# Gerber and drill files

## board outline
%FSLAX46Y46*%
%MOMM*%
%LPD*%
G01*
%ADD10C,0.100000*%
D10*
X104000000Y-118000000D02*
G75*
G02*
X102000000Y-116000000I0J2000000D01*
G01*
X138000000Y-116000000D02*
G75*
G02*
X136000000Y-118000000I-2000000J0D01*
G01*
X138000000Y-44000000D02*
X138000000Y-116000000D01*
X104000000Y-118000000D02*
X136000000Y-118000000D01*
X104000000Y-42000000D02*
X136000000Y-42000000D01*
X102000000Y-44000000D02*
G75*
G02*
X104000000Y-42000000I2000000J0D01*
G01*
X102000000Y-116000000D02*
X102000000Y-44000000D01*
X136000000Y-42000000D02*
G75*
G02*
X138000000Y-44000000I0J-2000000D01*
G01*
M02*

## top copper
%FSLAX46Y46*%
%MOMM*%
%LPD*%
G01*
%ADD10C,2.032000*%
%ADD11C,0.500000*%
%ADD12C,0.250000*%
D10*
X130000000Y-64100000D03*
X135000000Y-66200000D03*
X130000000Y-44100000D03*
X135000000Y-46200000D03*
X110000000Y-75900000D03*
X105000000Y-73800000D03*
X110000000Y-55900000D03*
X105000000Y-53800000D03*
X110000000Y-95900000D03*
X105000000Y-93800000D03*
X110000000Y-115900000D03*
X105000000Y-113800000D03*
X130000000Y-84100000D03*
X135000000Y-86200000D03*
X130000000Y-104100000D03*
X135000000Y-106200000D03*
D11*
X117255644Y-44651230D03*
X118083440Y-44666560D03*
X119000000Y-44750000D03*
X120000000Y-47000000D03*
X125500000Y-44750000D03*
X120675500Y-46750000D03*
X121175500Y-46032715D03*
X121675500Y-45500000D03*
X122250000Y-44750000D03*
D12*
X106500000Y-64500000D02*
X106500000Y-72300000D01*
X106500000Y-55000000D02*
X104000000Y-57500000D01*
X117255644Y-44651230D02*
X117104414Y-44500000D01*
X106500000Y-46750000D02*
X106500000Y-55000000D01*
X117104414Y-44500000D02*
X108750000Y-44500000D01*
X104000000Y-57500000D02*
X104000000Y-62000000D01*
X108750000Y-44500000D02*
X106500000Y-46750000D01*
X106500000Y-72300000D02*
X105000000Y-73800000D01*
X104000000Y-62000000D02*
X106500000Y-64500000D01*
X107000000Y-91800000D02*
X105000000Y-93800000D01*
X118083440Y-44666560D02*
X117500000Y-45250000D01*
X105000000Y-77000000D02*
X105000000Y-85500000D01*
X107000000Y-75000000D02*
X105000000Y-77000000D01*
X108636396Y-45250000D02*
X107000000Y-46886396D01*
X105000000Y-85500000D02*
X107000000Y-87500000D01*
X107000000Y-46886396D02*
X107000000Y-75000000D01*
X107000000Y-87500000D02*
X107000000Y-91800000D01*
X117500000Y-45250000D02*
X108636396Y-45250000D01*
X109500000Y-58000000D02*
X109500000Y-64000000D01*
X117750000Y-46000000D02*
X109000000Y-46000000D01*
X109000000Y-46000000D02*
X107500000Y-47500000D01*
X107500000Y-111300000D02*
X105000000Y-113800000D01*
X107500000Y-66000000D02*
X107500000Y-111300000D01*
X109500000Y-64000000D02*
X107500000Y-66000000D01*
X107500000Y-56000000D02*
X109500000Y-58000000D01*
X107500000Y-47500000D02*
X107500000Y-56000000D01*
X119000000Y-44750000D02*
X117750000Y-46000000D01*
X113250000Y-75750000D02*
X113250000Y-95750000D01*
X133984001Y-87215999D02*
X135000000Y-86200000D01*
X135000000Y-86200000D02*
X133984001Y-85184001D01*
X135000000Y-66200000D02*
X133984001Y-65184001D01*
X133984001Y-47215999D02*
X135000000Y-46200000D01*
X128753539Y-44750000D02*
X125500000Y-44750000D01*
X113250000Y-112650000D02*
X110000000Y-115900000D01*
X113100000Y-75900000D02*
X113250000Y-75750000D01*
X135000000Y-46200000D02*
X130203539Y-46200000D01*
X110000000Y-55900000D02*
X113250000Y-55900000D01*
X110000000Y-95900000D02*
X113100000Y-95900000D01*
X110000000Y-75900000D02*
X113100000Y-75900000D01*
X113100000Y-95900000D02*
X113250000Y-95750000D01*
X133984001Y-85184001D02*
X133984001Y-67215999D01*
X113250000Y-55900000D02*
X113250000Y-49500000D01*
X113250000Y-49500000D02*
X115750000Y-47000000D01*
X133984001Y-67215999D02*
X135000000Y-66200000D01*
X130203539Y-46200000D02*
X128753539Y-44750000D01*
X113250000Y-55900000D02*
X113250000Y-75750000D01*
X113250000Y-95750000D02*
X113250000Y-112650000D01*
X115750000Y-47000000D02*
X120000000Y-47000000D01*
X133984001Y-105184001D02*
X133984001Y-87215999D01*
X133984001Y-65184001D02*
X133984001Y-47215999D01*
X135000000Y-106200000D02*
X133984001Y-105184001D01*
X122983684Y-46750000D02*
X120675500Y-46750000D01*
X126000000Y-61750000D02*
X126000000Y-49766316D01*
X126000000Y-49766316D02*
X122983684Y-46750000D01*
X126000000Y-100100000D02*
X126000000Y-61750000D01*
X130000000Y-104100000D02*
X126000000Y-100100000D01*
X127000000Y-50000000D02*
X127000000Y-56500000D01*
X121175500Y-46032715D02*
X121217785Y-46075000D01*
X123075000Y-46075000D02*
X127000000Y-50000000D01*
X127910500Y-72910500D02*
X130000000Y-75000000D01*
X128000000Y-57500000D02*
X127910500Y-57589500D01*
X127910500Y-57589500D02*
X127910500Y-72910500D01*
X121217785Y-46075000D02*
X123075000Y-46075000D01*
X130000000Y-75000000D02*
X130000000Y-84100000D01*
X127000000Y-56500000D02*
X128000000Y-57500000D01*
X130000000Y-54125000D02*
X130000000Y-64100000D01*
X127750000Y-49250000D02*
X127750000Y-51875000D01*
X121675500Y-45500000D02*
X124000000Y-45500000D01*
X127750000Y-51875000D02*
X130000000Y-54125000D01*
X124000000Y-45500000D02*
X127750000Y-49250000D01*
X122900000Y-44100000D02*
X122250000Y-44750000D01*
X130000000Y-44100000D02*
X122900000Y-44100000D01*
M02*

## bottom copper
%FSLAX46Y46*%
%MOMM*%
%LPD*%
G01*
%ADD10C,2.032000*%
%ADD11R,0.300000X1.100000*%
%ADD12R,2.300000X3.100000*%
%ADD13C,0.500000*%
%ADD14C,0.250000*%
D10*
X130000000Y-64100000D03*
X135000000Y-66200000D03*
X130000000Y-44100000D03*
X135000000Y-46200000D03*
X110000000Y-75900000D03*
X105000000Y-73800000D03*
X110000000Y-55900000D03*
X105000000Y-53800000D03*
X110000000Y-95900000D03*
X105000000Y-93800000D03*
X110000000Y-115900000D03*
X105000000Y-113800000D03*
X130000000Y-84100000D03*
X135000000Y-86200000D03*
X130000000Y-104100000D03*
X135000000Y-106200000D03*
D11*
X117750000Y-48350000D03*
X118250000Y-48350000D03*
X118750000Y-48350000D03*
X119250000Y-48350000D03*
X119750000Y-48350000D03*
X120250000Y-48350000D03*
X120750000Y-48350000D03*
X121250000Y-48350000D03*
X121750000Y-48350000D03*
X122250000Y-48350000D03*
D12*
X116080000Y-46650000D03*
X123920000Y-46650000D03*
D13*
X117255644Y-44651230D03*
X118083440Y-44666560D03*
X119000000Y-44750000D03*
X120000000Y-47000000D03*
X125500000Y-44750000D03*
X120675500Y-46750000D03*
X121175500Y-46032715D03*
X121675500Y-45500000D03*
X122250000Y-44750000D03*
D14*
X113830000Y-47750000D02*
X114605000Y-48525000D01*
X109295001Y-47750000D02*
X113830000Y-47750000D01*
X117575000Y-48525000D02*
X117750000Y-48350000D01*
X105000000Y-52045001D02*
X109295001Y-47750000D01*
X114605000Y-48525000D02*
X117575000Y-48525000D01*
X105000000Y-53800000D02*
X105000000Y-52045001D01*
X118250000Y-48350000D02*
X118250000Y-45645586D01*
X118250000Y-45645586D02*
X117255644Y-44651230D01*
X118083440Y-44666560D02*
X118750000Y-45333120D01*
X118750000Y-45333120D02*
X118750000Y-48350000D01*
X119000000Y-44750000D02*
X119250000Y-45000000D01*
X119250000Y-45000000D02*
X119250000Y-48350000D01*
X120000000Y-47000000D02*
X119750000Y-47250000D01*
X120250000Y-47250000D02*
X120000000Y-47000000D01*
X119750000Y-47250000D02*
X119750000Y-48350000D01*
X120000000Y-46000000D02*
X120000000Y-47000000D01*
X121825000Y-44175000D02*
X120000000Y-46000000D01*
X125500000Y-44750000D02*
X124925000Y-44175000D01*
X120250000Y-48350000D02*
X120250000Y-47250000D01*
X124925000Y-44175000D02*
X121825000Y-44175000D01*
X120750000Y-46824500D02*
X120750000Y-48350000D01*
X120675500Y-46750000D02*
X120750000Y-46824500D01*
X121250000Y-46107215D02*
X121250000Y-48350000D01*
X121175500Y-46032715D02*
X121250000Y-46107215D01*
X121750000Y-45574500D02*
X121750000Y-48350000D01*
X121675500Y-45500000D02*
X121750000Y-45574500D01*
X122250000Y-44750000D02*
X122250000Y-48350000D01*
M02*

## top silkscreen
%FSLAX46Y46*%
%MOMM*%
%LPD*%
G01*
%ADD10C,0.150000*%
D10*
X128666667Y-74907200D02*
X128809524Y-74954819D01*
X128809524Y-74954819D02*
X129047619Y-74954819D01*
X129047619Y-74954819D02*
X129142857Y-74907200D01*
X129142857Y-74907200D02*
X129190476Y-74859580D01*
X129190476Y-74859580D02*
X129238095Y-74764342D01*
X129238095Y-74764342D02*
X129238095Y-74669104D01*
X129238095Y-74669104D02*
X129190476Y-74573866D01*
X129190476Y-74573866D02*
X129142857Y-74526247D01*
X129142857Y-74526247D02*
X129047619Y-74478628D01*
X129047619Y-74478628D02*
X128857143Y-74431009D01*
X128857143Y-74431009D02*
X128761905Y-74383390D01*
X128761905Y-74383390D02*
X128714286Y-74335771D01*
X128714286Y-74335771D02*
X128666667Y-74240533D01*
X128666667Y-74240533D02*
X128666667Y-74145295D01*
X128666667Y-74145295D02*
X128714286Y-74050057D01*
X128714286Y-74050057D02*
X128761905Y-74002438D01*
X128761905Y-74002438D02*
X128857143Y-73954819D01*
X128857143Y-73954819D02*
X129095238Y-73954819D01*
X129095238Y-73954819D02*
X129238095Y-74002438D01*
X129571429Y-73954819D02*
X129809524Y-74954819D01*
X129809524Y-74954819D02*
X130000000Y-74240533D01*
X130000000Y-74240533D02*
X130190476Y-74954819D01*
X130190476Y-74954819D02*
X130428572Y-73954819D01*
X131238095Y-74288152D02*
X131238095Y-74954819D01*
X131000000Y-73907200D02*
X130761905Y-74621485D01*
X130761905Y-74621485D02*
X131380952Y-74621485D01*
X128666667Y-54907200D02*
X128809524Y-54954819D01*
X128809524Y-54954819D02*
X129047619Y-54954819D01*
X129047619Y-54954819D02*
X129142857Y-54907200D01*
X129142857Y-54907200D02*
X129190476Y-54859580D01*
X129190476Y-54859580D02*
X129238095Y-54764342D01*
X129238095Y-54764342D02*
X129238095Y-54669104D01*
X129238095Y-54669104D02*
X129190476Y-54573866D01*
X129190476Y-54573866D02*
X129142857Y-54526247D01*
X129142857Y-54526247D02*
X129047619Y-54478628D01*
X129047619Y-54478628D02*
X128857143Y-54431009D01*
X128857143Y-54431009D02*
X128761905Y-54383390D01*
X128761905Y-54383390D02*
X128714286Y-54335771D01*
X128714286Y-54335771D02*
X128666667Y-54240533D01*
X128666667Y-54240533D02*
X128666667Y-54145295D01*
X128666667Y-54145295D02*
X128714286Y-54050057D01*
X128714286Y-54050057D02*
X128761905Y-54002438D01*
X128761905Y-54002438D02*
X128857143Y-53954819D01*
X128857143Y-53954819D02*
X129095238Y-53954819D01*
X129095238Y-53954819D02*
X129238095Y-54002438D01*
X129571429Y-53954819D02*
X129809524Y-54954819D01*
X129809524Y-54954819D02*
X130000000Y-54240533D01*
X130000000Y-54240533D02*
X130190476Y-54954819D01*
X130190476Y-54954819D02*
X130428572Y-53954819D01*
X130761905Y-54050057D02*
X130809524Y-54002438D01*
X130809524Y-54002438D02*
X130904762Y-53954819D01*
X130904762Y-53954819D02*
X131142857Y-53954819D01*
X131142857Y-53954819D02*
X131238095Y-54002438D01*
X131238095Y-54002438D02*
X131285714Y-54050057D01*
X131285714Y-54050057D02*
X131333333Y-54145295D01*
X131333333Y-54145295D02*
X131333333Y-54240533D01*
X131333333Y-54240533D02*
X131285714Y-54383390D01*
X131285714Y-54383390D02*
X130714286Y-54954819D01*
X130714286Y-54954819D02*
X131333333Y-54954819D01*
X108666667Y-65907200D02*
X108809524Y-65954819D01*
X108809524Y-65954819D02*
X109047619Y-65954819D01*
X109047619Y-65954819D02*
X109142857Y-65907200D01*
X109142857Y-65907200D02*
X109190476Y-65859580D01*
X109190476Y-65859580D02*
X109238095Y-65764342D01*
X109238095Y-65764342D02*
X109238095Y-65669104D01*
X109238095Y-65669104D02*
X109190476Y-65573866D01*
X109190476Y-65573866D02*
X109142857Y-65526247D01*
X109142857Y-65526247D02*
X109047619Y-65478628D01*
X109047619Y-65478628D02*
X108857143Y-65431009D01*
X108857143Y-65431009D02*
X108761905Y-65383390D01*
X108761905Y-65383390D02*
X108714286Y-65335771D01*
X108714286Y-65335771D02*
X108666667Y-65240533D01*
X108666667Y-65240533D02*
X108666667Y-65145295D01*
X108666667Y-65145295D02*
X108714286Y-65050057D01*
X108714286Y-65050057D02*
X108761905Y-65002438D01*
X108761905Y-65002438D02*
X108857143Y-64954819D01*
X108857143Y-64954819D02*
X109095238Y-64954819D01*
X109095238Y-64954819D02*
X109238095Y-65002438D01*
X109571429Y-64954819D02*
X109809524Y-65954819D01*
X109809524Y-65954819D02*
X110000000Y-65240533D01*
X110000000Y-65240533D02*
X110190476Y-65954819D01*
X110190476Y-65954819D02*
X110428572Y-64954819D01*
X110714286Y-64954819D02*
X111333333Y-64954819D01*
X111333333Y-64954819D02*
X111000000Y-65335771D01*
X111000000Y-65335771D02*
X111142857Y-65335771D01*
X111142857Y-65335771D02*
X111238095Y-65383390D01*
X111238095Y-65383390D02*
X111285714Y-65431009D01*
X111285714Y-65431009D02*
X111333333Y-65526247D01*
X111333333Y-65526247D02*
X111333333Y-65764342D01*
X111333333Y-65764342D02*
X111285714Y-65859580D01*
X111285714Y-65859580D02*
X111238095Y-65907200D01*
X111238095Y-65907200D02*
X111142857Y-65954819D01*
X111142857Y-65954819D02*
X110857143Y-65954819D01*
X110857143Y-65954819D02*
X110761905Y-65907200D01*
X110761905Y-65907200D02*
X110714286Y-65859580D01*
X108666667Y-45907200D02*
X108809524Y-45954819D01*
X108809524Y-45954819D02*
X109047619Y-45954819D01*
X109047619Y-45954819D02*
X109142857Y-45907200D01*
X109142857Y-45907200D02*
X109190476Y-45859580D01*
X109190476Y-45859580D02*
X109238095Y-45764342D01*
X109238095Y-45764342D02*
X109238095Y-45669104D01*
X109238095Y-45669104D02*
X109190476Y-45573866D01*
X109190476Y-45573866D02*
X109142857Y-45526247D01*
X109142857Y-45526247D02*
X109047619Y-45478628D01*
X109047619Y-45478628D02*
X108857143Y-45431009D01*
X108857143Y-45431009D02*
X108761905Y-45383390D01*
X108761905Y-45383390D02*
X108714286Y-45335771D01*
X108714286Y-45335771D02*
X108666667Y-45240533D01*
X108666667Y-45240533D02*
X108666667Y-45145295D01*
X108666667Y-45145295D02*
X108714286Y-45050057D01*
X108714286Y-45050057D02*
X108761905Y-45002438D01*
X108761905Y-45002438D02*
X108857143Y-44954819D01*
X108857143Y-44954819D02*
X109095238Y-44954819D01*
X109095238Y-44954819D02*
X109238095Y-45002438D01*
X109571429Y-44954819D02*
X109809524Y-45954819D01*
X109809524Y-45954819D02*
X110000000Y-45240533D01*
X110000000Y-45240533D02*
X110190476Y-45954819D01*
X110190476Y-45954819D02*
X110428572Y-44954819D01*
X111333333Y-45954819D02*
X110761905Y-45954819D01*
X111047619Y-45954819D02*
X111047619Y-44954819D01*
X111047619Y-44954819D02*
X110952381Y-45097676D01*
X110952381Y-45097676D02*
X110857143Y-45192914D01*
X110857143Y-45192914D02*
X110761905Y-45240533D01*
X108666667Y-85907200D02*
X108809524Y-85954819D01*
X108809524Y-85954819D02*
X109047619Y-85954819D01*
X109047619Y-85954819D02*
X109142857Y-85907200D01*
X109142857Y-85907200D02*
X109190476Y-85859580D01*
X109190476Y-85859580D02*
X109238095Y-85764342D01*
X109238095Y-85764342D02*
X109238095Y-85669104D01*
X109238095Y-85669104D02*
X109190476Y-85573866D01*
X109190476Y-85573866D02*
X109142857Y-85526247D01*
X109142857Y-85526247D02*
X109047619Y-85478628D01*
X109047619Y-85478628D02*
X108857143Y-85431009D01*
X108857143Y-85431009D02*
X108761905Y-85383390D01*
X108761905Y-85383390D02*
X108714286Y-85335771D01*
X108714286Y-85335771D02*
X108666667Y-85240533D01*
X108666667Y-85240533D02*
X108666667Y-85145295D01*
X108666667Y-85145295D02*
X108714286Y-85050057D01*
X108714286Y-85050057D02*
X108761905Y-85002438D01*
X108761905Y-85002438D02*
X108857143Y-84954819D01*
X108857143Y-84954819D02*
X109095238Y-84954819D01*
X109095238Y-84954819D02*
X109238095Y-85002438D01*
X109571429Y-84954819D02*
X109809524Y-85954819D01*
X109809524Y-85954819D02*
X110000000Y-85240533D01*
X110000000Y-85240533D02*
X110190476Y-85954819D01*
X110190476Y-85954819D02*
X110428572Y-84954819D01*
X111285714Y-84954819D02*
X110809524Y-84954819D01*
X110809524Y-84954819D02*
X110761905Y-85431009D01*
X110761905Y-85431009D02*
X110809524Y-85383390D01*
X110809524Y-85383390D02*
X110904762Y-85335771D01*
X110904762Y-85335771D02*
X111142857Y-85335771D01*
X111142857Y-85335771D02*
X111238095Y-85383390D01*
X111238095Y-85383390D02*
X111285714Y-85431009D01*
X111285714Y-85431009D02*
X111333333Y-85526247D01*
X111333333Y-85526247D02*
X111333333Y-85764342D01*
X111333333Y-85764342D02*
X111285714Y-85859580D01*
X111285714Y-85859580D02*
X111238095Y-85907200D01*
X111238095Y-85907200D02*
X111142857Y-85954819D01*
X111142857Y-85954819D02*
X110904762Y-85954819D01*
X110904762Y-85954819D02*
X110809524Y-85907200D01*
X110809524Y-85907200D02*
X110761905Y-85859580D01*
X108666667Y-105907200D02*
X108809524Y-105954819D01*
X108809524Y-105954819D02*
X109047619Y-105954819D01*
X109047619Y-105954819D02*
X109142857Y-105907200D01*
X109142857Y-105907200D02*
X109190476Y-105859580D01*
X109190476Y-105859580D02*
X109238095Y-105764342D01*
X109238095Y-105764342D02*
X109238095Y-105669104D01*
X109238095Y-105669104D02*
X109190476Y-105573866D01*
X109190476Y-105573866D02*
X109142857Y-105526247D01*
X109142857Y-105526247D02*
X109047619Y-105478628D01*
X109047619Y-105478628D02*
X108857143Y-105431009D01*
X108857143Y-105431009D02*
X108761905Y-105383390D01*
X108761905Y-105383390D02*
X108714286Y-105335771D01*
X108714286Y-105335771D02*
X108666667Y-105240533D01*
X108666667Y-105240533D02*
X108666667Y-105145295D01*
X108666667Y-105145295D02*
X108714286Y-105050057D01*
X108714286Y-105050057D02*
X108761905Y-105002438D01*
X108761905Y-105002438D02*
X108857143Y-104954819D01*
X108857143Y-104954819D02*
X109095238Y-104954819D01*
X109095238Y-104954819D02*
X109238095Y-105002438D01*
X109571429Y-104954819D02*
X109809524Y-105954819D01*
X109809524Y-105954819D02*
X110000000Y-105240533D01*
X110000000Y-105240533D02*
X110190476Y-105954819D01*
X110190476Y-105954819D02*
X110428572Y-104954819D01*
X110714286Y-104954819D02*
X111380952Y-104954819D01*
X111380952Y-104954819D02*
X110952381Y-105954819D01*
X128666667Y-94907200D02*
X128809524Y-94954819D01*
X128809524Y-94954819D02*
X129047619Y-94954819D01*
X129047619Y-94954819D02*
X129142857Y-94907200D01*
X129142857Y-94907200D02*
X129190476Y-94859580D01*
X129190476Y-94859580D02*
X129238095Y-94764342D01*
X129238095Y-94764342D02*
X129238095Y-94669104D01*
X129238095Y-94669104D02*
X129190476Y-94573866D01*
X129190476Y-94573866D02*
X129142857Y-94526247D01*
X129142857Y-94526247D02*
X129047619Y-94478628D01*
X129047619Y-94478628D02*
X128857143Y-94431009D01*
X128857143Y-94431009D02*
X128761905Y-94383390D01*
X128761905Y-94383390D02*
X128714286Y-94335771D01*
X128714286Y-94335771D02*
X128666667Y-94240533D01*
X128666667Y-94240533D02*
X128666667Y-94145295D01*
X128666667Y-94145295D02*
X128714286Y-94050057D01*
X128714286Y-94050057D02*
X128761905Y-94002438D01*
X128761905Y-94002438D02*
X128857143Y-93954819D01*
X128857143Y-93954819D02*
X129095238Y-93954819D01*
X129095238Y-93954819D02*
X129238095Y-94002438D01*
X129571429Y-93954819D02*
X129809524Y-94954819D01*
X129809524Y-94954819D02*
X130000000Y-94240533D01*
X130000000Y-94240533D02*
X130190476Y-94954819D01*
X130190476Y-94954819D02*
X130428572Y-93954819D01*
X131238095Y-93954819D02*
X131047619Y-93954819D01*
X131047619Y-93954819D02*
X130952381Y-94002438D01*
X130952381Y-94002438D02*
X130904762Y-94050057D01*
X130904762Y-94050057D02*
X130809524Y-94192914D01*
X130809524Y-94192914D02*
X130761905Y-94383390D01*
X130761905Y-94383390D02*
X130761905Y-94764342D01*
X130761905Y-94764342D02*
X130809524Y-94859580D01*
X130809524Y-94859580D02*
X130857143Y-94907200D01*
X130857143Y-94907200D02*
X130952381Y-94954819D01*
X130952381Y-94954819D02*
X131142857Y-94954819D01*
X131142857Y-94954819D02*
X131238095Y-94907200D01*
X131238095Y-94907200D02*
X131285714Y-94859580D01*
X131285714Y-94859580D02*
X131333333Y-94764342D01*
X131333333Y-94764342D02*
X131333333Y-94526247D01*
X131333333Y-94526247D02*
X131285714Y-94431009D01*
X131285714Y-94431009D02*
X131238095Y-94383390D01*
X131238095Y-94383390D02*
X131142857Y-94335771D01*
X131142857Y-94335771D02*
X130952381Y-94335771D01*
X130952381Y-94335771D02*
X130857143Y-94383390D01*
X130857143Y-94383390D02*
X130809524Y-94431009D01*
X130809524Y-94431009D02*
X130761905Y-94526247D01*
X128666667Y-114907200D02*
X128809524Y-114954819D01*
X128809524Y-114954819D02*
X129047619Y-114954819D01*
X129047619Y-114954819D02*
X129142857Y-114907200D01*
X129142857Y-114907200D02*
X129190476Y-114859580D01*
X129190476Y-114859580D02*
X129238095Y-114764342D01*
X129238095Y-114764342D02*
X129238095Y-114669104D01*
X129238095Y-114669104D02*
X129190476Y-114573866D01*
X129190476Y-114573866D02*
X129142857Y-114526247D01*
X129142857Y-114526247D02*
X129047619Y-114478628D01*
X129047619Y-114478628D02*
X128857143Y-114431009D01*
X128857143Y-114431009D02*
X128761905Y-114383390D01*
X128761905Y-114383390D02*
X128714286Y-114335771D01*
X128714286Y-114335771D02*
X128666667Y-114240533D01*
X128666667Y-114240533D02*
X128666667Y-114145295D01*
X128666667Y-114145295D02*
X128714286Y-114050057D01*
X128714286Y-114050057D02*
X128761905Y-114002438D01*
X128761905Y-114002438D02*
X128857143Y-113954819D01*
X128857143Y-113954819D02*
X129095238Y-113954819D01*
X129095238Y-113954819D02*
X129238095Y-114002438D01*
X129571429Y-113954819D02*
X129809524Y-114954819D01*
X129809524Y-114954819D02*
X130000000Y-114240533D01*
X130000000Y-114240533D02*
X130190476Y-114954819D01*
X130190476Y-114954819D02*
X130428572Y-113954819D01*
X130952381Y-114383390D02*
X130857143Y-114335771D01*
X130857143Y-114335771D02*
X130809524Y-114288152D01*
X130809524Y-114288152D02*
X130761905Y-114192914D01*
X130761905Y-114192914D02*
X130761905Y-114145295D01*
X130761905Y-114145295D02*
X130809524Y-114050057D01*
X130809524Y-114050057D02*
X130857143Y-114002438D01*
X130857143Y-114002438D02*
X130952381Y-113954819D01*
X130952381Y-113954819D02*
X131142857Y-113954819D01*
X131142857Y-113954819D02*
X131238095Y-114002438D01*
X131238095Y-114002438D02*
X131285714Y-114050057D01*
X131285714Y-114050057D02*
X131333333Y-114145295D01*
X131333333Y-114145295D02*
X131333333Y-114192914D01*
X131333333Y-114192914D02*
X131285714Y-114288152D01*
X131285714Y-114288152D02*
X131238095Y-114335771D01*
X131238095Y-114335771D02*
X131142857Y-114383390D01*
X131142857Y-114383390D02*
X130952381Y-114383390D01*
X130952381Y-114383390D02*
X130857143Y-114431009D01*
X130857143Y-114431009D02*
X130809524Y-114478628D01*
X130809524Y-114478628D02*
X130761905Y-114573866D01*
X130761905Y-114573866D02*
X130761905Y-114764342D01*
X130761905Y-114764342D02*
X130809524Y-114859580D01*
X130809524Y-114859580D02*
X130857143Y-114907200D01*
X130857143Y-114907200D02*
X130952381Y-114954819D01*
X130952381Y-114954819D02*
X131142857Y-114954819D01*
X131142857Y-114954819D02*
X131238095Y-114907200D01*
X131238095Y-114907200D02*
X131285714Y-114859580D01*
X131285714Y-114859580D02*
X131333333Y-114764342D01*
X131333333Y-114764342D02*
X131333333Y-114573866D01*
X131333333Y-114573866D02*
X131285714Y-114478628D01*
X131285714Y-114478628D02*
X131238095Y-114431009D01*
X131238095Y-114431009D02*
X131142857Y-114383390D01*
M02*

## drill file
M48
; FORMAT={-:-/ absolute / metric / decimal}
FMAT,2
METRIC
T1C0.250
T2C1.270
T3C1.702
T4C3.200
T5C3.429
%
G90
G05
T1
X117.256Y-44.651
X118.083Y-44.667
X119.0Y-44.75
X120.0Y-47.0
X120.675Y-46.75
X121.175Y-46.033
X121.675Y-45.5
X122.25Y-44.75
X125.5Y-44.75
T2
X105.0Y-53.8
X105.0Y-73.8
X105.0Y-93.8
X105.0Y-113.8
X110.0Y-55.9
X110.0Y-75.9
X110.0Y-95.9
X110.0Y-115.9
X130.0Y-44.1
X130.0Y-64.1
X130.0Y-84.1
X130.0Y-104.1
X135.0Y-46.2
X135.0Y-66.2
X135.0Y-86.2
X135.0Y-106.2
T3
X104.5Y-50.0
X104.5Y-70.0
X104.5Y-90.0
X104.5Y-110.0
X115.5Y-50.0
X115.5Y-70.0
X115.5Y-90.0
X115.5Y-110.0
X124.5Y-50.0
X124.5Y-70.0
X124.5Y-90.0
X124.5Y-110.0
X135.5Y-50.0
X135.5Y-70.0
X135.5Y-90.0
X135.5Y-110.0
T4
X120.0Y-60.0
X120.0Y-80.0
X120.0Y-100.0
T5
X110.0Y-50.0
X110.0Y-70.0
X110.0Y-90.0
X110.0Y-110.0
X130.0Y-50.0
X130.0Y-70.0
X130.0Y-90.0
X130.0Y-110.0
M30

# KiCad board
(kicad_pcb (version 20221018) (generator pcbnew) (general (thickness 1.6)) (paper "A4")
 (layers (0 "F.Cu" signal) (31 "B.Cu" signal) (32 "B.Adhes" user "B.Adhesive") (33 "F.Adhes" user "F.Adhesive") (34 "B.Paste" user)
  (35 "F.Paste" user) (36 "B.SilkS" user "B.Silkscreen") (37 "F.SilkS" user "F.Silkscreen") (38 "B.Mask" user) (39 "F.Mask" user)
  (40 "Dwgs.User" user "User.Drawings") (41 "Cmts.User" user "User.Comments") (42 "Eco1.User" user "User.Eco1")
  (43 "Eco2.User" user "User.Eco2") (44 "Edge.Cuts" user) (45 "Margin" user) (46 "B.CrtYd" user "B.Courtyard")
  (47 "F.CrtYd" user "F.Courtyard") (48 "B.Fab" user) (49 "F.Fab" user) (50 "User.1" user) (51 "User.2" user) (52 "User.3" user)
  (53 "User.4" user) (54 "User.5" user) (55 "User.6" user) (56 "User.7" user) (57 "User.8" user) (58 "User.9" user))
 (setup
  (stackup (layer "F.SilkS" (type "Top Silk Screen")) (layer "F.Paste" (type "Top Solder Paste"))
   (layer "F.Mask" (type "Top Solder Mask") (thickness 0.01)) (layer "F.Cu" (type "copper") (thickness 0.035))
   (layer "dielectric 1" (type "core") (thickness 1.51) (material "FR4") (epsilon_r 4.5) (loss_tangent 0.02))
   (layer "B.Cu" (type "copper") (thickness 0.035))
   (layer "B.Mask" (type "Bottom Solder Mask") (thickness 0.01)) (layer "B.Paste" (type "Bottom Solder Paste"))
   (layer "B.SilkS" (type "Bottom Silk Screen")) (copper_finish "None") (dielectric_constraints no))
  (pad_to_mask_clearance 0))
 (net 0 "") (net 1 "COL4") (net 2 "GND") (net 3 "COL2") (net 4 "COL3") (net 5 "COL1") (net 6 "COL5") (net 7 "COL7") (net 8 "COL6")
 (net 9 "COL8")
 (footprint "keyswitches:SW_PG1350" (layer "F.Cu") (at 130 70 180)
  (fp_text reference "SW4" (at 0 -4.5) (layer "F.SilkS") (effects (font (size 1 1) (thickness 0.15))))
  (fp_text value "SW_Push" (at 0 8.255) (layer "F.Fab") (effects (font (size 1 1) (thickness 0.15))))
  (pad "" np_thru_hole circle (at -5.5 0 180) (size 1.7018 1.7018) (drill 1.7018) (layers "*.Cu" "*.Mask"))
  (pad "" np_thru_hole circle (at 0 0 180) (size 3.429 3.429) (drill 3.429) (layers "*.Cu" "*.Mask"))
  (pad "" np_thru_hole circle (at 5.5 0 180) (size 1.7018 1.7018) (drill 1.7018) (layers "*.Cu" "*.Mask"))
  (pad "1" thru_hole circle (at 0 5.9 180) (size 2.032 2.032) (drill 1.27) (layers "*.Cu" "*.Mask") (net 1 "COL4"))
  (pad "2" thru_hole circle (at -5 3.8 180) (size 2.032 2.032) (drill 1.27) (layers "*.Cu" "*.Mask") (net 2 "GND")))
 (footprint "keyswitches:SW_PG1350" (layer "F.Cu") (at 130 50 180)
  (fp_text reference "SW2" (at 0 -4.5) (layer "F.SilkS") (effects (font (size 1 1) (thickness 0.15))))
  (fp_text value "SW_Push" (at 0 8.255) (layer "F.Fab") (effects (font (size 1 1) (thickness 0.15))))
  (pad "" np_thru_hole circle (at -5.5 0 180) (size 1.7018 1.7018) (drill 1.7018) (layers "*.Cu" "*.Mask"))
  (pad "" np_thru_hole circle (at 0 0 180) (size 3.429 3.429) (drill 3.429) (layers "*.Cu" "*.Mask"))
  (pad "" np_thru_hole circle (at 5.5 0 180) (size 1.7018 1.7018) (drill 1.7018) (layers "*.Cu" "*.Mask"))
  (pad "1" thru_hole circle (at 0 5.9 180) (size 2.032 2.032) (drill 1.27) (layers "*.Cu" "*.Mask") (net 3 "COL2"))
  (pad "2" thru_hole circle (at -5 3.8 180) (size 2.032 2.032) (drill 1.27) (layers "*.Cu" "*.Mask") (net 2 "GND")))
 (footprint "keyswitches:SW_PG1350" (layer "F.Cu") (at 110 70)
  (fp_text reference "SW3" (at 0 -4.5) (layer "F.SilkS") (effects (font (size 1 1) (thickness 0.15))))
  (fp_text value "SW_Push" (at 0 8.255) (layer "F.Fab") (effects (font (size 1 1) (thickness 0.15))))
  (pad "" np_thru_hole circle (at -5.5 0) (size 1.7018 1.7018) (drill 1.7018) (layers "*.Cu" "*.Mask"))
  (pad "" np_thru_hole circle (at 0 0) (size 3.429 3.429) (drill 3.429) (layers "*.Cu" "*.Mask"))
  (pad "" np_thru_hole circle (at 5.5 0) (size 1.7018 1.7018) (drill 1.7018) (layers "*.Cu" "*.Mask"))
  (pad "1" thru_hole circle (at 0 5.9) (size 2.032 2.032) (drill 1.27) (layers "*.Cu" "*.Mask") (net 2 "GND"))
  (pad "2" thru_hole circle (at -5 3.8) (size 2.032 2.032) (drill 1.27) (layers "*.Cu" "*.Mask") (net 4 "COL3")))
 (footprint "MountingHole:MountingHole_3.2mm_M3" (layer "F.Cu") (at 120 100)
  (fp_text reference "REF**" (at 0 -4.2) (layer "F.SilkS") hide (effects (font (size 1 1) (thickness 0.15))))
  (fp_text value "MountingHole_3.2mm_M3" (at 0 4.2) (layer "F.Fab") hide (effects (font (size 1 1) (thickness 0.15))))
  (pad "" np_thru_hole circle (at 0 0) (size 3.2 3.2) (drill 3.2) (layers "*.Cu" "*.Mask")))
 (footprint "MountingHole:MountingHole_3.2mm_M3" (layer "F.Cu") (at 120 80)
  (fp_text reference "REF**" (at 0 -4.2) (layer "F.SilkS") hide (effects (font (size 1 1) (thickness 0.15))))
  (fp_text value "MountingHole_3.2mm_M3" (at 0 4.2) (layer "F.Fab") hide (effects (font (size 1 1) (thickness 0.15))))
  (pad "" np_thru_hole circle (at 0 0) (size 3.2 3.2) (drill 3.2) (layers "*.Cu" "*.Mask")))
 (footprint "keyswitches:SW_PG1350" (layer "F.Cu") (at 110 50)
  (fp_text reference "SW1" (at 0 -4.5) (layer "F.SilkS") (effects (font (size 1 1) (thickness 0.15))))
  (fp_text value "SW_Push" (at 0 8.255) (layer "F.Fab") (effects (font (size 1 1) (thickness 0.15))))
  (pad "" np_thru_hole circle (at -5.5 0) (size 1.7018 1.7018) (drill 1.7018) (layers "*.Cu" "*.Mask"))
  (pad "" np_thru_hole circle (at 0 0) (size 3.429 3.429) (drill 3.429) (layers "*.Cu" "*.Mask"))
  (pad "" np_thru_hole circle (at 5.5 0) (size 1.7018 1.7018) (drill 1.7018) (layers "*.Cu" "*.Mask"))
  (pad "1" thru_hole circle (at 0 5.9) (size 2.032 2.032) (drill 1.27) (layers "*.Cu" "*.Mask") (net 2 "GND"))
  (pad "2" thru_hole circle (at -5 3.8) (size 2.032 2.032) (drill 1.27) (layers "*.Cu" "*.Mask") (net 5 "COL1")))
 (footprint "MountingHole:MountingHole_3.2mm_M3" (layer "F.Cu") (at 120 60)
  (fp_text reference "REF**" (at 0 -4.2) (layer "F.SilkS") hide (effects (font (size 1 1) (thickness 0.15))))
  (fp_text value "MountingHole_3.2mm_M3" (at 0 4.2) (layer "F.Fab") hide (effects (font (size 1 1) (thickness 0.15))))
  (pad "" np_thru_hole circle (at 0 0) (size 3.2 3.2) (drill 3.2) (layers "*.Cu" "*.Mask")))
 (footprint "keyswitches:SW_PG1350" (layer "F.Cu") (at 110 90)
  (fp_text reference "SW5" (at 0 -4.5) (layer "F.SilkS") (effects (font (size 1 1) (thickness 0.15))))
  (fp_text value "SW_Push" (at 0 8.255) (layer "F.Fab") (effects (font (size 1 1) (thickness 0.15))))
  (pad "" np_thru_hole circle (at -5.5 0) (size 1.7018 1.7018) (drill 1.7018) (layers "*.Cu" "*.Mask"))
  (pad "" np_thru_hole circle (at 0 0) (size 3.429 3.429) (drill 3.429) (layers "*.Cu" "*.Mask"))
  (pad "" np_thru_hole circle (at 5.5 0) (size 1.7018 1.7018) (drill 1.7018) (layers "*.Cu" "*.Mask"))
  (pad "1" thru_hole circle (at 0 5.9) (size 2.032 2.032) (drill 1.27) (layers "*.Cu" "*.Mask") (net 2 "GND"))
  (pad "2" thru_hole circle (at -5 3.8) (size 2.032 2.032) (drill 1.27) (layers "*.Cu" "*.Mask") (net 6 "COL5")))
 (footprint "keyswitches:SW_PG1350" (layer "F.Cu") (at 110 110)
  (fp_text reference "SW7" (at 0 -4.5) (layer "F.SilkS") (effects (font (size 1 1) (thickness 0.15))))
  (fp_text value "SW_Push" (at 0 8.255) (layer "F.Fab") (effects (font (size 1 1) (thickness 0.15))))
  (pad "" np_thru_hole circle (at -5.5 0) (size 1.7018 1.7018) (drill 1.7018) (layers "*.Cu" "*.Mask"))
  (pad "" np_thru_hole circle (at 0 0) (size 3.429 3.429) (drill 3.429) (layers "*.Cu" "*.Mask"))
  (pad "" np_thru_hole circle (at 5.5 0) (size 1.7018 1.7018) (drill 1.7018) (layers "*.Cu" "*.Mask"))
  (pad "1" thru_hole circle (at 0 5.9) (size 2.032 2.032) (drill 1.27) (layers "*.Cu" "*.Mask") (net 2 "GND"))
  (pad "2" thru_hole circle (at -5 3.8) (size 2.032 2.032) (drill 1.27) (layers "*.Cu" "*.Mask") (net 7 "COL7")))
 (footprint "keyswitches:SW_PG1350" (layer "F.Cu") (at 130 90 180)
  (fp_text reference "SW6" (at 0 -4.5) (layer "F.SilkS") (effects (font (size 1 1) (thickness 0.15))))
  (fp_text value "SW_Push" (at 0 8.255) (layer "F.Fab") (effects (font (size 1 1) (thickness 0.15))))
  (pad "" np_thru_hole circle (at -5.5 0 180) (size 1.7018 1.7018) (drill 1.7018) (layers "*.Cu" "*.Mask"))
  (pad "" np_thru_hole circle (at 0 0 180) (size 3.429 3.429) (drill 3.429) (layers "*.Cu" "*.Mask"))
  (pad "" np_thru_hole circle (at 5.5 0 180) (size 1.7018 1.7018) (drill 1.7018) (layers "*.Cu" "*.Mask"))
  (pad "1" thru_hole circle (at 0 5.9 180) (size 2.032 2.032) (drill 1.27) (layers "*.Cu" "*.Mask") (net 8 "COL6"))
  (pad "2" thru_hole circle (at -5 3.8 180) (size 2.032 2.032) (drill 1.27) (layers "*.Cu" "*.Mask") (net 2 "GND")))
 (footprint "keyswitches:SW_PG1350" (layer "F.Cu") (at 130 110 180)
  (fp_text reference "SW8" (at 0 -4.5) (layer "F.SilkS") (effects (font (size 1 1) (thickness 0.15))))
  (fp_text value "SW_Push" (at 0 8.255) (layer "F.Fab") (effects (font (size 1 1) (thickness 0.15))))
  (pad "" np_thru_hole circle (at -5.5 0 180) (size 1.7018 1.7018) (drill 1.7018) (layers "*.Cu" "*.Mask"))
  (pad "" np_thru_hole circle (at 0 0 180) (size 3.429 3.429) (drill 3.429) (layers "*.Cu" "*.Mask"))
  (pad "" np_thru_hole circle (at 5.5 0 180) (size 1.7018 1.7018) (drill 1.7018) (layers "*.Cu" "*.Mask"))
  (pad "1" thru_hole circle (at 0 5.9 180) (size 2.032 2.032) (drill 1.27) (layers "*.Cu" "*.Mask") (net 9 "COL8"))
  (pad "2" thru_hole circle (at -5 3.8 180) (size 2.032 2.032) (drill 1.27) (layers "*.Cu" "*.Mask") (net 2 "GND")))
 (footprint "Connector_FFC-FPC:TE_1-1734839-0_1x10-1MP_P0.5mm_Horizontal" (layer "B.Cu") (at 120 47)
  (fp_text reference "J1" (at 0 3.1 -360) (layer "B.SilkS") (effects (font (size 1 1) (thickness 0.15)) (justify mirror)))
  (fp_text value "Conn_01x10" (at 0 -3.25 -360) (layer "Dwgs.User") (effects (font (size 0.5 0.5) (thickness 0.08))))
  (pad "1" smd rect (at -2.25 1.35) (size 0.3 1.1) (layers "B.Cu" "B.Paste" "B.Mask") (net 5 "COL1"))
  (pad "2" smd rect (at -1.75 1.35) (size 0.3 1.1) (layers "B.Cu" "B.Paste" "B.Mask") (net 4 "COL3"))
  (pad "3" smd rect (at -1.25 1.35) (size 0.3 1.1) (layers "B.Cu" "B.Paste" "B.Mask") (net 6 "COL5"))
  (pad "4" smd rect (at -0.75 1.35) (size 0.3 1.1) (layers "B.Cu" "B.Paste" "B.Mask") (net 7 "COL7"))
  (pad "5" smd rect (at -0.25 1.35) (size 0.3 1.1) (layers "B.Cu" "B.Paste" "B.Mask") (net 2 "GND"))
  (pad "6" smd rect (at 0.25 1.35) (size 0.3 1.1) (layers "B.Cu" "B.Paste" "B.Mask") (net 2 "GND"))
  (pad "7" smd rect (at 0.75 1.35) (size 0.3 1.1) (layers "B.Cu" "B.Paste" "B.Mask") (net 9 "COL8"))
  (pad "8" smd rect (at 1.25 1.35) (size 0.3 1.1) (layers "B.Cu" "B.Paste" "B.Mask") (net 8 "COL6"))
  (pad "9" smd rect (at 1.75 1.35) (size 0.3 1.1) (layers "B.Cu" "B.Paste" "B.Mask") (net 1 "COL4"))
  (pad "10" smd rect (at 2.25 1.35) (size 0.3 1.1) (layers "B.Cu" "B.Paste" "B.Mask") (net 3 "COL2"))
  (pad "MP" smd rect (at -3.92 -0.35) (size 2.3 3.1) (layers "B.Cu" "B.Paste" "B.Mask"))
  (pad "MP" smd rect (at 3.92 -0.35) (size 2.3 3.1) (layers "B.Cu" "B.Paste" "B.Mask")))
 (gr_arc (start 104 118) (mid 102.585786 117.414214) (end 102 116) (stroke (width 0.1) (type default)) (layer "Edge.Cuts"))
 (gr_arc (start 138 116) (mid 137.414214 117.414214) (end 136 118) (stroke (width 0.1) (type default)) (layer "Edge.Cuts"))
 (gr_line (start 138 44) (end 138 116) (stroke (width 0.1) (type default)) (layer "Edge.Cuts"))
 (gr_line (start 104 118) (end 136 118) (stroke (width 0.1) (type default)) (layer "Edge.Cuts"))
 (gr_line (start 104 42) (end 136 42) (stroke (width 0.1) (type default)) (layer "Edge.Cuts"))
 (gr_arc (start 102 44) (mid 102.585786 42.585786) (end 104 42) (stroke (width 0.1) (type default)) (layer "Edge.Cuts"))
 (gr_line (start 102 116) (end 102 44) (stroke (width 0.1) (type default)) (layer "Edge.Cuts"))
 (gr_arc (start 136 42) (mid 137.414214 42.585786) (end 138 44) (stroke (width 0.1) (type default)) (layer "Edge.Cuts"))
 (segment (start 113.83 47.75) (end 114.605 48.525) (width 0.25) (layer "B.Cu") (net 5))
 (segment (start 109.295001 47.75) (end 113.83 47.75) (width 0.25) (layer "B.Cu") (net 5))
 (segment (start 117.575 48.525) (end 117.75 48.35) (width 0.25) (layer "B.Cu") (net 5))
 (segment (start 105 52.045001) (end 109.295001 47.75) (width 0.25) (layer "B.Cu") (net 5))
 (segment (start 114.605 48.525) (end 117.575 48.525) (width 0.25) (layer "B.Cu") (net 5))
 (segment (start 105 53.8) (end 105 52.045001) (width 0.25) (layer "B.Cu") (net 5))
 (segment (start 106.5 64.5) (end 106.5 72.3) (width 0.25) (layer "F.Cu") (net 4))
 (segment (start 106.5 55) (end 104 57.5) (width 0.25) (layer "F.Cu") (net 4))
 (segment (start 117.255644 44.65123) (end 117.104414 44.5) (width 0.25) (layer "F.Cu") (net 4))
 (segment (start 106.5 46.75) (end 106.5 55) (width 0.25) (layer "F.Cu") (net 4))
 (segment (start 117.104414 44.5) (end 108.75 44.5) (width 0.25) (layer "F.Cu") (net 4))
 (segment (start 104 57.5) (end 104 62) (width 0.25) (layer "F.Cu") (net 4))
 (segment (start 108.75 44.5) (end 106.5 46.75) (width 0.25) (layer "F.Cu") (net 4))
 (segment (start 106.5 72.3) (end 105 73.8) (width 0.25) (layer "F.Cu") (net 4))
 (segment (start 104 62) (end 106.5 64.5) (width 0.25) (layer "F.Cu") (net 4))
 (via (at 117.255644 44.65123) (size 0.5) (drill 0.25) (layers "F.Cu" "B.Cu") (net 4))
 (segment (start 118.25 48.35) (end 118.25 45.645586) (width 0.25) (layer "B.Cu") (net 4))
 (segment (start 118.25 45.645586) (end 117.255644 44.65123) (width 0.25) (layer "B.Cu") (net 4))
 (segment (start 107 91.8) (end 105 93.8) (width 0.25) (layer "F.Cu") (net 6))
 (segment (start 118.08344 44.66656) (end 117.5 45.25) (width 0.25) (layer "F.Cu") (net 6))
 (segment (start 105 77) (end 105 85.5) (width 0.25) (layer "F.Cu") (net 6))
 (segment (start 107 75) (end 105 77) (width 0.25) (layer "F.Cu") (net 6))
 (segment (start 108.636396 45.25) (end 107 46.886396) (width 0.25) (layer "F.Cu") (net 6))
 (segment (start 105 85.5) (end 107 87.5) (width 0.25) (layer "F.Cu") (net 6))
 (segment (start 107 46.886396) (end 107 75) (width 0.25) (layer "F.Cu") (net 6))
 (segment (start 107 87.5) (end 107 91.8) (width 0.25) (layer "F.Cu") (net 6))
 (segment (start 117.5 45.25) (end 108.636396 45.25) (width 0.25) (layer "F.Cu") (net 6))
 (via (at 118.08344 44.66656) (size 0.5) (drill 0.25) (layers "F.Cu" "B.Cu") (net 6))
 (segment (start 118.08344 44.66656) (end 118.75 45.33312) (width 0.25) (layer "B.Cu") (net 6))
 (segment (start 118.75 45.33312) (end 118.75 48.35) (width 0.25) (layer "B.Cu") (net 6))
 (segment (start 109.5 58) (end 109.5 64) (width 0.25) (layer "F.Cu") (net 7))
 (segment (start 117.75 46) (end 109 46) (width 0.25) (layer "F.Cu") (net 7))
 (segment (start 109 46) (end 107.5 47.5) (width 0.25) (layer "F.Cu") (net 7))
 (segment (start 107.5 111.3) (end 105 113.8) (width 0.25) (layer "F.Cu") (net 7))
 (segment (start 107.5 66) (end 107.5 111.3) (width 0.25) (layer "F.Cu") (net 7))
 (segment (start 109.5 64) (end 107.5 66) (width 0.25) (layer "F.Cu") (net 7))
 (segment (start 107.5 56) (end 109.5 58) (width 0.25) (layer "F.Cu") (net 7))
 (segment (start 107.5 47.5) (end 107.5 56) (width 0.25) (layer "F.Cu") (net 7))
 (segment (start 119 44.75) (end 117.75 46) (width 0.25) (layer "F.Cu") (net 7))
 (via (at 119 44.75) (size 0.5) (drill 0.25) (layers "F.Cu" "B.Cu") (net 7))
 (segment (start 119 44.75) (end 119.25 45) (width 0.25) (layer "B.Cu") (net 7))
 (segment (start 119.25 45) (end 119.25 48.35) (width 0.25) (layer "B.Cu") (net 7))
 (segment (start 113.25 75.75) (end 113.25 95.75) (width 0.25) (layer "F.Cu") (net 2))
 (segment (start 133.984001 87.215999) (end 135 86.2) (width 0.25) (layer "F.Cu") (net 2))
 (segment (start 135 86.2) (end 133.984001 85.184001) (width 0.25) (layer "F.Cu") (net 2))
 (segment (start 135 66.2) (end 133.984001 65.184001) (width 0.25) (layer "F.Cu") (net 2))
 (segment (start 133.984001 47.215999) (end 135 46.2) (width 0.25) (layer "F.Cu") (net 2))
 (segment (start 128.753539 44.75) (end 125.5 44.75) (width 0.25) (layer "F.Cu") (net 2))
 (segment (start 113.25 112.65) (end 110 115.9) (width 0.25) (layer "F.Cu") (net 2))
 (segment (start 113.1 75.9) (end 113.25 75.75) (width 0.25) (layer "F.Cu") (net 2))
 (segment (start 135 46.2) (end 130.203539 46.2) (width 0.25) (layer "F.Cu") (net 2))
 (segment (start 110 55.9) (end 113.25 55.9) (width 0.25) (layer "F.Cu") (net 2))
 (segment (start 110 95.9) (end 113.1 95.9) (width 0.25) (layer "F.Cu") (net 2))
 (segment (start 110 75.9) (end 113.1 75.9) (width 0.25) (layer "F.Cu") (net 2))
 (segment (start 113.1 95.9) (end 113.25 95.75) (width 0.25) (layer "F.Cu") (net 2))
 (segment (start 133.984001 85.184001) (end 133.984001 67.215999) (width 0.25) (layer "F.Cu") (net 2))
 (segment (start 113.25 55.9) (end 113.25 49.5) (width 0.25) (layer "F.Cu") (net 2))
 (segment (start 113.25 49.5) (end 115.75 47) (width 0.25) (layer "F.Cu") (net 2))
 (segment (start 133.984001 67.215999) (end 135 66.2) (width 0.25) (layer "F.Cu") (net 2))
 (segment (start 130.203539 46.2) (end 128.753539 44.75) (width 0.25) (layer "F.Cu") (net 2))
 (segment (start 113.25 55.9) (end 113.25 75.75) (width 0.25) (layer "F.Cu") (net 2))
 (segment (start 113.25 95.75) (end 113.25 112.65) (width 0.25) (layer "F.Cu") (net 2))
 (segment (start 115.75 47) (end 120 47) (width 0.25) (layer "F.Cu") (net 2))
 (segment (start 133.984001 105.184001) (end 133.984001 87.215999) (width 0.25) (layer "F.Cu") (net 2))
 (segment (start 133.984001 65.184001) (end 133.984001 47.215999) (width 0.25) (layer "F.Cu") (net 2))
 (segment (start 135 106.2) (end 133.984001 105.184001) (width 0.25) (layer "F.Cu") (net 2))
 (via (at 120 47) (size 0.5) (drill 0.25) (layers "F.Cu" "B.Cu") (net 2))
 (via (at 125.5 44.75) (size 0.5) (drill 0.25) (layers "F.Cu" "B.Cu") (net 2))
 (segment (start 120 47) (end 119.75 47.25) (width 0.25) (layer "B.Cu") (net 2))
 (segment (start 120.25 47.25) (end 120 47) (width 0.25) (layer "B.Cu") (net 2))
 (segment (start 119.75 47.25) (end 119.75 48.35) (width 0.25) (layer "B.Cu") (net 2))
 (segment (start 120 46) (end 120 47) (width 0.25) (layer "B.Cu") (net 2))
 (segment (start 121.825 44.175) (end 120 46) (width 0.25) (layer "B.Cu") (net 2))
 (segment (start 125.5 44.75) (end 124.925 44.175) (width 0.25) (layer "B.Cu") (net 2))
 (segment (start 120.25 48.35) (end 120.25 47.25) (width 0.25) (layer "B.Cu") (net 2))
 (segment (start 124.925 44.175) (end 121.825 44.175) (width 0.25) (layer "B.Cu") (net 2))
 (segment (start 122.983684 46.75) (end 120.6755 46.75) (width 0.25) (layer "F.Cu") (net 9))
 (segment (start 126 61.75) (end 126 49.766316) (width 0.25) (layer "F.Cu") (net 9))
 (segment (start 126 49.766316) (end 122.983684 46.75) (width 0.25) (layer "F.Cu") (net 9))
 (segment (start 126 100.1) (end 126 61.75) (width 0.25) (layer "F.Cu") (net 9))
 (segment (start 130 104.1) (end 126 100.1) (width 0.25) (layer "F.Cu") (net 9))
 (via (at 120.6755 46.75) (size 0.5) (drill 0.25) (layers "F.Cu" "B.Cu") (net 9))
 (segment (start 120.75 46.8245) (end 120.75 48.35) (width 0.25) (layer "B.Cu") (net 9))
 (segment (start 120.6755 46.75) (end 120.75 46.8245) (width 0.25) (layer "B.Cu") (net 9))
 (segment (start 127 50) (end 127 56.5) (width 0.25) (layer "F.Cu") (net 8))
 (segment (start 121.1755 46.032715) (end 121.217785 46.075) (width 0.25) (layer "F.Cu") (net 8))
 (segment (start 123.075 46.075) (end 127 50) (width 0.25) (layer "F.Cu") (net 8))
 (segment (start 127.9105 72.9105) (end 130 75) (width 0.25) (layer "F.Cu") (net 8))
 (segment (start 128 57.5) (end 127.9105 57.5895) (width 0.25) (layer "F.Cu") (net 8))
 (segment (start 127.9105 57.5895) (end 127.9105 72.9105) (width 0.25) (layer "F.Cu") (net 8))
 (segment (start 121.217785 46.075) (end 123.075 46.075) (width 0.25) (layer "F.Cu") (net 8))
 (segment (start 130 75) (end 130 84.1) (width 0.25) (layer "F.Cu") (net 8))
 (segment (start 127 56.5) (end 128 57.5) (width 0.25) (layer "F.Cu") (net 8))
 (via (at 121.1755 46.032715) (size 0.5) (drill 0.25) (layers "F.Cu" "B.Cu") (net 8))
 (segment (start 121.25 46.107215) (end 121.25 48.35) (width 0.25) (layer "B.Cu") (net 8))
 (segment (start 121.1755 46.032715) (end 121.25 46.107215) (width 0.25) (layer "B.Cu") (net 8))
 (segment (start 130 54.125) (end 130 64.1) (width 0.25) (layer "F.Cu") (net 1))
 (segment (start 127.75 49.25) (end 127.75 51.875) (width 0.25) (layer "F.Cu") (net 1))
 (segment (start 121.6755 45.5) (end 124 45.5) (width 0.25) (layer "F.Cu") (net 1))
 (segment (start 127.75 51.875) (end 130 54.125) (width 0.25) (layer "F.Cu") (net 1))
 (segment (start 124 45.5) (end 127.75 49.25) (width 0.25) (layer "F.Cu") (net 1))
 (via (at 121.6755 45.5) (size 0.5) (drill 0.25) (layers "F.Cu" "B.Cu") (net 1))
 (segment (start 121.75 45.5745) (end 121.75 48.35) (width 0.25) (layer "B.Cu") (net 1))
 (segment (start 121.6755 45.5) (end 121.75 45.5745) (width 0.25) (layer "B.Cu") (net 1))
 (segment (start 122.9 44.1) (end 122.25 44.75) (width 0.25) (layer "F.Cu") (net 3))
 (segment (start 130 44.1) (end 122.9 44.1) (width 0.25) (layer "F.Cu") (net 3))
 (via (at 122.25 44.75) (size 0.5) (drill 0.25) (layers "F.Cu" "B.Cu") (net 3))
 (segment (start 122.25 44.75) (end 122.25 48.35) (width 0.25) (layer "B.Cu") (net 3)))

